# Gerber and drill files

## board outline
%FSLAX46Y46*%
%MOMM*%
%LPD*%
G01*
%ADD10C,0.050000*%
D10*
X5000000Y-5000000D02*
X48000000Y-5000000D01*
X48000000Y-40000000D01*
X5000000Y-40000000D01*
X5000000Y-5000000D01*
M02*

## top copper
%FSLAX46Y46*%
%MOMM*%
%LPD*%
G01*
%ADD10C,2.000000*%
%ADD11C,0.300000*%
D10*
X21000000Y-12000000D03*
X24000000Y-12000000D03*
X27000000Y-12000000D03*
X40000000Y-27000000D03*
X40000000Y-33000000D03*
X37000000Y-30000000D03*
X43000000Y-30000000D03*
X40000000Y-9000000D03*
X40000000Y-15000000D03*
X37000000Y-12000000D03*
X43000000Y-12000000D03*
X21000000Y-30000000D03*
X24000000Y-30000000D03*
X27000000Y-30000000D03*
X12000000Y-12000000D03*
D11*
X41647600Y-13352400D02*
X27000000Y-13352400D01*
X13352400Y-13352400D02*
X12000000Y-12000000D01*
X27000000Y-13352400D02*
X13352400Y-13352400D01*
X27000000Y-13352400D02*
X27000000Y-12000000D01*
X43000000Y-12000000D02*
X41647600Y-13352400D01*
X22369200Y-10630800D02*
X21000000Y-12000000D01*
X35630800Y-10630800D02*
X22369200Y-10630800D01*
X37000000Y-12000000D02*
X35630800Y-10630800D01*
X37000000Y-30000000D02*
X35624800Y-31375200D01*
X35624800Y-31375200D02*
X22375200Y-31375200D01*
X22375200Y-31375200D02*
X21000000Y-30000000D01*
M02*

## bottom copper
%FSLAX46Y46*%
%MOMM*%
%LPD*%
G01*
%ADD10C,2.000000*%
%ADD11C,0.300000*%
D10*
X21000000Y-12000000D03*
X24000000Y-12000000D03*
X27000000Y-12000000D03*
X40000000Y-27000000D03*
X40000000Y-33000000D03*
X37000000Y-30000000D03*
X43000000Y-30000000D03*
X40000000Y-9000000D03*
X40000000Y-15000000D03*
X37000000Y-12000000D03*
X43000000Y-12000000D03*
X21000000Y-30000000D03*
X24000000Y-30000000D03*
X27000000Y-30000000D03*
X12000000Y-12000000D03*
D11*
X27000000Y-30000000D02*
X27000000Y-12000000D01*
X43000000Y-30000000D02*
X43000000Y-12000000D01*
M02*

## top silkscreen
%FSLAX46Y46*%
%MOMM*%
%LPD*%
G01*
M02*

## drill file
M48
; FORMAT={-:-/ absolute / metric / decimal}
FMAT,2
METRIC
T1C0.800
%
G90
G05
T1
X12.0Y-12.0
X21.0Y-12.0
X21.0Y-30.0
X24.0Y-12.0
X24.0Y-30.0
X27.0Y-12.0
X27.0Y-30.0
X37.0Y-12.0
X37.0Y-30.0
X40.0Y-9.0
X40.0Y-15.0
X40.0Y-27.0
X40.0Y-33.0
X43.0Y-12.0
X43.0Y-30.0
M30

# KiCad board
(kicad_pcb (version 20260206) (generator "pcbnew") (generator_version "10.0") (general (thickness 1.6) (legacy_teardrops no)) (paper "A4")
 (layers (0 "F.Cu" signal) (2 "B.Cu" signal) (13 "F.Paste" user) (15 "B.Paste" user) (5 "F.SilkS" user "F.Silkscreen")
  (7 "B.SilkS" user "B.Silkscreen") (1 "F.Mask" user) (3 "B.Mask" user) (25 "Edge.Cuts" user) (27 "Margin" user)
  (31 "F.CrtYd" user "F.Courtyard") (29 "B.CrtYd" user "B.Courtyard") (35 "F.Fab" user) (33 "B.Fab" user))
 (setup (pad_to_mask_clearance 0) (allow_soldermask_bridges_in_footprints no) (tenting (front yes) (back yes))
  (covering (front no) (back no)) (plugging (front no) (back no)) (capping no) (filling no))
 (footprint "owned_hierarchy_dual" (layer "F.Cu") (at 24 12)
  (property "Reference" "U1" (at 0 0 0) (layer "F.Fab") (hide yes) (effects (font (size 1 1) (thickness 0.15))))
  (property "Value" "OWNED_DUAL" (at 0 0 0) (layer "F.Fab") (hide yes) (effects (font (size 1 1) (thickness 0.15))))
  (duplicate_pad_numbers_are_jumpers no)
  (pad "1" thru_hole circle (at -3 0) (size 2 2) (drill 0.8) (layers "*.Cu" "*.Mask") (remove_unused_layers no) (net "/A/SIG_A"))
  (pad "2" thru_hole circle (at 0 0) (size 2 2) (drill 0.8) (layers "*.Cu" "*.Mask") (remove_unused_layers no) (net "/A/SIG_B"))
  (pad "3" thru_hole circle (at 3 0) (size 2 2) (drill 0.8) (layers "*.Cu" "*.Mask") (remove_unused_layers no) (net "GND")))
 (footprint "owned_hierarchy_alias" (layer "F.Cu") (at 40 30)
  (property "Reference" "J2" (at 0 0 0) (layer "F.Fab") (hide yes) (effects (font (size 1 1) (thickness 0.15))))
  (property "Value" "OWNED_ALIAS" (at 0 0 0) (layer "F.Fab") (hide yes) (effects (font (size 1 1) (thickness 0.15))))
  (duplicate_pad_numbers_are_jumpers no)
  (pad "MP" thru_hole circle (at 0 -3) (size 2 2) (drill 0.8) (layers "*.Cu" "*.Mask") (remove_unused_layers no))
  (pad "MP" thru_hole circle (at 0 3) (size 2 2) (drill 0.8) (layers "*.Cu" "*.Mask") (remove_unused_layers no))
  (pad "R" thru_hole circle (at -3 0) (size 2 2) (drill 0.8) (layers "*.Cu" "*.Mask") (remove_unused_layers no) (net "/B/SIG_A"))
  (pad "T" thru_hole circle (at 3 0) (size 2 2) (drill 0.8) (layers "*.Cu" "*.Mask") (remove_unused_layers no) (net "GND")))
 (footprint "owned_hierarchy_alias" (layer "F.Cu") (at 40 12)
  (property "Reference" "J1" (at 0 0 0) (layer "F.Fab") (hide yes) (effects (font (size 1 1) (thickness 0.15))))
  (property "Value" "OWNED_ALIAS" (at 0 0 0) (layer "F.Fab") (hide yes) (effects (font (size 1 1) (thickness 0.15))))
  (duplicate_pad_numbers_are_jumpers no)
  (pad "MP" thru_hole circle (at 0 -3) (size 2 2) (drill 0.8) (layers "*.Cu" "*.Mask") (remove_unused_layers no))
  (pad "MP" thru_hole circle (at 0 3) (size 2 2) (drill 0.8) (layers "*.Cu" "*.Mask") (remove_unused_layers no))
  (pad "R" thru_hole circle (at -3 0) (size 2 2) (drill 0.8) (layers "*.Cu" "*.Mask") (remove_unused_layers no) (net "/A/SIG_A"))
  (pad "T" thru_hole circle (at 3 0) (size 2 2) (drill 0.8) (layers "*.Cu" "*.Mask") (remove_unused_layers no) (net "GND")))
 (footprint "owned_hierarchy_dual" (layer "F.Cu") (at 24 30)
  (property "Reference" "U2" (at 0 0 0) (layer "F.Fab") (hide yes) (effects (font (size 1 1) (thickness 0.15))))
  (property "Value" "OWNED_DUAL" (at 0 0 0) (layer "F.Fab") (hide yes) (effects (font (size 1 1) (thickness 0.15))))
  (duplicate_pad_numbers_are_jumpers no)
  (pad "1" thru_hole circle (at -3 0) (size 2 2) (drill 0.8) (layers "*.Cu" "*.Mask") (remove_unused_layers no) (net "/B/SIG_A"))
  (pad "2" thru_hole circle (at 0 0) (size 2 2) (drill 0.8) (layers "*.Cu" "*.Mask") (remove_unused_layers no) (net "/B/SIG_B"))
  (pad "3" thru_hole circle (at 3 0) (size 2 2) (drill 0.8) (layers "*.Cu" "*.Mask") (remove_unused_layers no) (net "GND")))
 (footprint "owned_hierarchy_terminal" (layer "F.Cu") (at 12 12)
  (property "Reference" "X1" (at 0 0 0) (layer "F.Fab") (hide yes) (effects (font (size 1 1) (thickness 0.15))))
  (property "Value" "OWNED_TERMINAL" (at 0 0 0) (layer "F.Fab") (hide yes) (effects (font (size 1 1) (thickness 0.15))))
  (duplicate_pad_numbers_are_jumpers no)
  (pad "1" thru_hole circle (at 0 0) (size 2 2) (drill 0.8) (layers "*.Cu" "*.Mask") (remove_unused_layers no) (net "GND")))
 (gr_rect (start 5 5) (end 48 40) (stroke (width 0.05) (type default)) (fill no) (layer "Edge.Cuts"))
 (segment (start 41.6476 13.3524) (end 27 13.3524) (width 0.3) (layer "F.Cu") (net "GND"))
 (segment (start 13.3524 13.3524) (end 12 12) (width 0.3) (layer "F.Cu") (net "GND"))
 (segment (start 27 13.3524) (end 13.3524 13.3524) (width 0.3) (layer "F.Cu") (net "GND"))
 (segment (start 27 13.3524) (end 27 12) (width 0.3) (layer "F.Cu") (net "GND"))
 (segment (start 43 12) (end 41.6476 13.3524) (width 0.3) (layer "F.Cu") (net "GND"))
 (segment (start 27 30) (end 27 12) (width 0.3) (layer "B.Cu") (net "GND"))
 (segment (start 43 30) (end 43 12) (width 0.3) (layer "B.Cu") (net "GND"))
 (segment (start 22.3692 10.6308) (end 21 12) (width 0.3) (layer "F.Cu") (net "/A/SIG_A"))
 (segment (start 35.6308 10.6308) (end 22.3692 10.6308) (width 0.3) (layer "F.Cu") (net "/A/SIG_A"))
 (segment (start 37 12) (end 35.6308 10.6308) (width 0.3) (layer "F.Cu") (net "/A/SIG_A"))
 (segment (start 37 30) (end 35.6248 31.3752) (width 0.3) (layer "F.Cu") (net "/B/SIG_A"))
 (segment (start 35.6248 31.3752) (end 22.3752 31.3752) (width 0.3) (layer "F.Cu") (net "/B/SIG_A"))
 (segment (start 22.3752 31.3752) (end 21 30) (width 0.3) (layer "F.Cu") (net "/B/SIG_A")))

